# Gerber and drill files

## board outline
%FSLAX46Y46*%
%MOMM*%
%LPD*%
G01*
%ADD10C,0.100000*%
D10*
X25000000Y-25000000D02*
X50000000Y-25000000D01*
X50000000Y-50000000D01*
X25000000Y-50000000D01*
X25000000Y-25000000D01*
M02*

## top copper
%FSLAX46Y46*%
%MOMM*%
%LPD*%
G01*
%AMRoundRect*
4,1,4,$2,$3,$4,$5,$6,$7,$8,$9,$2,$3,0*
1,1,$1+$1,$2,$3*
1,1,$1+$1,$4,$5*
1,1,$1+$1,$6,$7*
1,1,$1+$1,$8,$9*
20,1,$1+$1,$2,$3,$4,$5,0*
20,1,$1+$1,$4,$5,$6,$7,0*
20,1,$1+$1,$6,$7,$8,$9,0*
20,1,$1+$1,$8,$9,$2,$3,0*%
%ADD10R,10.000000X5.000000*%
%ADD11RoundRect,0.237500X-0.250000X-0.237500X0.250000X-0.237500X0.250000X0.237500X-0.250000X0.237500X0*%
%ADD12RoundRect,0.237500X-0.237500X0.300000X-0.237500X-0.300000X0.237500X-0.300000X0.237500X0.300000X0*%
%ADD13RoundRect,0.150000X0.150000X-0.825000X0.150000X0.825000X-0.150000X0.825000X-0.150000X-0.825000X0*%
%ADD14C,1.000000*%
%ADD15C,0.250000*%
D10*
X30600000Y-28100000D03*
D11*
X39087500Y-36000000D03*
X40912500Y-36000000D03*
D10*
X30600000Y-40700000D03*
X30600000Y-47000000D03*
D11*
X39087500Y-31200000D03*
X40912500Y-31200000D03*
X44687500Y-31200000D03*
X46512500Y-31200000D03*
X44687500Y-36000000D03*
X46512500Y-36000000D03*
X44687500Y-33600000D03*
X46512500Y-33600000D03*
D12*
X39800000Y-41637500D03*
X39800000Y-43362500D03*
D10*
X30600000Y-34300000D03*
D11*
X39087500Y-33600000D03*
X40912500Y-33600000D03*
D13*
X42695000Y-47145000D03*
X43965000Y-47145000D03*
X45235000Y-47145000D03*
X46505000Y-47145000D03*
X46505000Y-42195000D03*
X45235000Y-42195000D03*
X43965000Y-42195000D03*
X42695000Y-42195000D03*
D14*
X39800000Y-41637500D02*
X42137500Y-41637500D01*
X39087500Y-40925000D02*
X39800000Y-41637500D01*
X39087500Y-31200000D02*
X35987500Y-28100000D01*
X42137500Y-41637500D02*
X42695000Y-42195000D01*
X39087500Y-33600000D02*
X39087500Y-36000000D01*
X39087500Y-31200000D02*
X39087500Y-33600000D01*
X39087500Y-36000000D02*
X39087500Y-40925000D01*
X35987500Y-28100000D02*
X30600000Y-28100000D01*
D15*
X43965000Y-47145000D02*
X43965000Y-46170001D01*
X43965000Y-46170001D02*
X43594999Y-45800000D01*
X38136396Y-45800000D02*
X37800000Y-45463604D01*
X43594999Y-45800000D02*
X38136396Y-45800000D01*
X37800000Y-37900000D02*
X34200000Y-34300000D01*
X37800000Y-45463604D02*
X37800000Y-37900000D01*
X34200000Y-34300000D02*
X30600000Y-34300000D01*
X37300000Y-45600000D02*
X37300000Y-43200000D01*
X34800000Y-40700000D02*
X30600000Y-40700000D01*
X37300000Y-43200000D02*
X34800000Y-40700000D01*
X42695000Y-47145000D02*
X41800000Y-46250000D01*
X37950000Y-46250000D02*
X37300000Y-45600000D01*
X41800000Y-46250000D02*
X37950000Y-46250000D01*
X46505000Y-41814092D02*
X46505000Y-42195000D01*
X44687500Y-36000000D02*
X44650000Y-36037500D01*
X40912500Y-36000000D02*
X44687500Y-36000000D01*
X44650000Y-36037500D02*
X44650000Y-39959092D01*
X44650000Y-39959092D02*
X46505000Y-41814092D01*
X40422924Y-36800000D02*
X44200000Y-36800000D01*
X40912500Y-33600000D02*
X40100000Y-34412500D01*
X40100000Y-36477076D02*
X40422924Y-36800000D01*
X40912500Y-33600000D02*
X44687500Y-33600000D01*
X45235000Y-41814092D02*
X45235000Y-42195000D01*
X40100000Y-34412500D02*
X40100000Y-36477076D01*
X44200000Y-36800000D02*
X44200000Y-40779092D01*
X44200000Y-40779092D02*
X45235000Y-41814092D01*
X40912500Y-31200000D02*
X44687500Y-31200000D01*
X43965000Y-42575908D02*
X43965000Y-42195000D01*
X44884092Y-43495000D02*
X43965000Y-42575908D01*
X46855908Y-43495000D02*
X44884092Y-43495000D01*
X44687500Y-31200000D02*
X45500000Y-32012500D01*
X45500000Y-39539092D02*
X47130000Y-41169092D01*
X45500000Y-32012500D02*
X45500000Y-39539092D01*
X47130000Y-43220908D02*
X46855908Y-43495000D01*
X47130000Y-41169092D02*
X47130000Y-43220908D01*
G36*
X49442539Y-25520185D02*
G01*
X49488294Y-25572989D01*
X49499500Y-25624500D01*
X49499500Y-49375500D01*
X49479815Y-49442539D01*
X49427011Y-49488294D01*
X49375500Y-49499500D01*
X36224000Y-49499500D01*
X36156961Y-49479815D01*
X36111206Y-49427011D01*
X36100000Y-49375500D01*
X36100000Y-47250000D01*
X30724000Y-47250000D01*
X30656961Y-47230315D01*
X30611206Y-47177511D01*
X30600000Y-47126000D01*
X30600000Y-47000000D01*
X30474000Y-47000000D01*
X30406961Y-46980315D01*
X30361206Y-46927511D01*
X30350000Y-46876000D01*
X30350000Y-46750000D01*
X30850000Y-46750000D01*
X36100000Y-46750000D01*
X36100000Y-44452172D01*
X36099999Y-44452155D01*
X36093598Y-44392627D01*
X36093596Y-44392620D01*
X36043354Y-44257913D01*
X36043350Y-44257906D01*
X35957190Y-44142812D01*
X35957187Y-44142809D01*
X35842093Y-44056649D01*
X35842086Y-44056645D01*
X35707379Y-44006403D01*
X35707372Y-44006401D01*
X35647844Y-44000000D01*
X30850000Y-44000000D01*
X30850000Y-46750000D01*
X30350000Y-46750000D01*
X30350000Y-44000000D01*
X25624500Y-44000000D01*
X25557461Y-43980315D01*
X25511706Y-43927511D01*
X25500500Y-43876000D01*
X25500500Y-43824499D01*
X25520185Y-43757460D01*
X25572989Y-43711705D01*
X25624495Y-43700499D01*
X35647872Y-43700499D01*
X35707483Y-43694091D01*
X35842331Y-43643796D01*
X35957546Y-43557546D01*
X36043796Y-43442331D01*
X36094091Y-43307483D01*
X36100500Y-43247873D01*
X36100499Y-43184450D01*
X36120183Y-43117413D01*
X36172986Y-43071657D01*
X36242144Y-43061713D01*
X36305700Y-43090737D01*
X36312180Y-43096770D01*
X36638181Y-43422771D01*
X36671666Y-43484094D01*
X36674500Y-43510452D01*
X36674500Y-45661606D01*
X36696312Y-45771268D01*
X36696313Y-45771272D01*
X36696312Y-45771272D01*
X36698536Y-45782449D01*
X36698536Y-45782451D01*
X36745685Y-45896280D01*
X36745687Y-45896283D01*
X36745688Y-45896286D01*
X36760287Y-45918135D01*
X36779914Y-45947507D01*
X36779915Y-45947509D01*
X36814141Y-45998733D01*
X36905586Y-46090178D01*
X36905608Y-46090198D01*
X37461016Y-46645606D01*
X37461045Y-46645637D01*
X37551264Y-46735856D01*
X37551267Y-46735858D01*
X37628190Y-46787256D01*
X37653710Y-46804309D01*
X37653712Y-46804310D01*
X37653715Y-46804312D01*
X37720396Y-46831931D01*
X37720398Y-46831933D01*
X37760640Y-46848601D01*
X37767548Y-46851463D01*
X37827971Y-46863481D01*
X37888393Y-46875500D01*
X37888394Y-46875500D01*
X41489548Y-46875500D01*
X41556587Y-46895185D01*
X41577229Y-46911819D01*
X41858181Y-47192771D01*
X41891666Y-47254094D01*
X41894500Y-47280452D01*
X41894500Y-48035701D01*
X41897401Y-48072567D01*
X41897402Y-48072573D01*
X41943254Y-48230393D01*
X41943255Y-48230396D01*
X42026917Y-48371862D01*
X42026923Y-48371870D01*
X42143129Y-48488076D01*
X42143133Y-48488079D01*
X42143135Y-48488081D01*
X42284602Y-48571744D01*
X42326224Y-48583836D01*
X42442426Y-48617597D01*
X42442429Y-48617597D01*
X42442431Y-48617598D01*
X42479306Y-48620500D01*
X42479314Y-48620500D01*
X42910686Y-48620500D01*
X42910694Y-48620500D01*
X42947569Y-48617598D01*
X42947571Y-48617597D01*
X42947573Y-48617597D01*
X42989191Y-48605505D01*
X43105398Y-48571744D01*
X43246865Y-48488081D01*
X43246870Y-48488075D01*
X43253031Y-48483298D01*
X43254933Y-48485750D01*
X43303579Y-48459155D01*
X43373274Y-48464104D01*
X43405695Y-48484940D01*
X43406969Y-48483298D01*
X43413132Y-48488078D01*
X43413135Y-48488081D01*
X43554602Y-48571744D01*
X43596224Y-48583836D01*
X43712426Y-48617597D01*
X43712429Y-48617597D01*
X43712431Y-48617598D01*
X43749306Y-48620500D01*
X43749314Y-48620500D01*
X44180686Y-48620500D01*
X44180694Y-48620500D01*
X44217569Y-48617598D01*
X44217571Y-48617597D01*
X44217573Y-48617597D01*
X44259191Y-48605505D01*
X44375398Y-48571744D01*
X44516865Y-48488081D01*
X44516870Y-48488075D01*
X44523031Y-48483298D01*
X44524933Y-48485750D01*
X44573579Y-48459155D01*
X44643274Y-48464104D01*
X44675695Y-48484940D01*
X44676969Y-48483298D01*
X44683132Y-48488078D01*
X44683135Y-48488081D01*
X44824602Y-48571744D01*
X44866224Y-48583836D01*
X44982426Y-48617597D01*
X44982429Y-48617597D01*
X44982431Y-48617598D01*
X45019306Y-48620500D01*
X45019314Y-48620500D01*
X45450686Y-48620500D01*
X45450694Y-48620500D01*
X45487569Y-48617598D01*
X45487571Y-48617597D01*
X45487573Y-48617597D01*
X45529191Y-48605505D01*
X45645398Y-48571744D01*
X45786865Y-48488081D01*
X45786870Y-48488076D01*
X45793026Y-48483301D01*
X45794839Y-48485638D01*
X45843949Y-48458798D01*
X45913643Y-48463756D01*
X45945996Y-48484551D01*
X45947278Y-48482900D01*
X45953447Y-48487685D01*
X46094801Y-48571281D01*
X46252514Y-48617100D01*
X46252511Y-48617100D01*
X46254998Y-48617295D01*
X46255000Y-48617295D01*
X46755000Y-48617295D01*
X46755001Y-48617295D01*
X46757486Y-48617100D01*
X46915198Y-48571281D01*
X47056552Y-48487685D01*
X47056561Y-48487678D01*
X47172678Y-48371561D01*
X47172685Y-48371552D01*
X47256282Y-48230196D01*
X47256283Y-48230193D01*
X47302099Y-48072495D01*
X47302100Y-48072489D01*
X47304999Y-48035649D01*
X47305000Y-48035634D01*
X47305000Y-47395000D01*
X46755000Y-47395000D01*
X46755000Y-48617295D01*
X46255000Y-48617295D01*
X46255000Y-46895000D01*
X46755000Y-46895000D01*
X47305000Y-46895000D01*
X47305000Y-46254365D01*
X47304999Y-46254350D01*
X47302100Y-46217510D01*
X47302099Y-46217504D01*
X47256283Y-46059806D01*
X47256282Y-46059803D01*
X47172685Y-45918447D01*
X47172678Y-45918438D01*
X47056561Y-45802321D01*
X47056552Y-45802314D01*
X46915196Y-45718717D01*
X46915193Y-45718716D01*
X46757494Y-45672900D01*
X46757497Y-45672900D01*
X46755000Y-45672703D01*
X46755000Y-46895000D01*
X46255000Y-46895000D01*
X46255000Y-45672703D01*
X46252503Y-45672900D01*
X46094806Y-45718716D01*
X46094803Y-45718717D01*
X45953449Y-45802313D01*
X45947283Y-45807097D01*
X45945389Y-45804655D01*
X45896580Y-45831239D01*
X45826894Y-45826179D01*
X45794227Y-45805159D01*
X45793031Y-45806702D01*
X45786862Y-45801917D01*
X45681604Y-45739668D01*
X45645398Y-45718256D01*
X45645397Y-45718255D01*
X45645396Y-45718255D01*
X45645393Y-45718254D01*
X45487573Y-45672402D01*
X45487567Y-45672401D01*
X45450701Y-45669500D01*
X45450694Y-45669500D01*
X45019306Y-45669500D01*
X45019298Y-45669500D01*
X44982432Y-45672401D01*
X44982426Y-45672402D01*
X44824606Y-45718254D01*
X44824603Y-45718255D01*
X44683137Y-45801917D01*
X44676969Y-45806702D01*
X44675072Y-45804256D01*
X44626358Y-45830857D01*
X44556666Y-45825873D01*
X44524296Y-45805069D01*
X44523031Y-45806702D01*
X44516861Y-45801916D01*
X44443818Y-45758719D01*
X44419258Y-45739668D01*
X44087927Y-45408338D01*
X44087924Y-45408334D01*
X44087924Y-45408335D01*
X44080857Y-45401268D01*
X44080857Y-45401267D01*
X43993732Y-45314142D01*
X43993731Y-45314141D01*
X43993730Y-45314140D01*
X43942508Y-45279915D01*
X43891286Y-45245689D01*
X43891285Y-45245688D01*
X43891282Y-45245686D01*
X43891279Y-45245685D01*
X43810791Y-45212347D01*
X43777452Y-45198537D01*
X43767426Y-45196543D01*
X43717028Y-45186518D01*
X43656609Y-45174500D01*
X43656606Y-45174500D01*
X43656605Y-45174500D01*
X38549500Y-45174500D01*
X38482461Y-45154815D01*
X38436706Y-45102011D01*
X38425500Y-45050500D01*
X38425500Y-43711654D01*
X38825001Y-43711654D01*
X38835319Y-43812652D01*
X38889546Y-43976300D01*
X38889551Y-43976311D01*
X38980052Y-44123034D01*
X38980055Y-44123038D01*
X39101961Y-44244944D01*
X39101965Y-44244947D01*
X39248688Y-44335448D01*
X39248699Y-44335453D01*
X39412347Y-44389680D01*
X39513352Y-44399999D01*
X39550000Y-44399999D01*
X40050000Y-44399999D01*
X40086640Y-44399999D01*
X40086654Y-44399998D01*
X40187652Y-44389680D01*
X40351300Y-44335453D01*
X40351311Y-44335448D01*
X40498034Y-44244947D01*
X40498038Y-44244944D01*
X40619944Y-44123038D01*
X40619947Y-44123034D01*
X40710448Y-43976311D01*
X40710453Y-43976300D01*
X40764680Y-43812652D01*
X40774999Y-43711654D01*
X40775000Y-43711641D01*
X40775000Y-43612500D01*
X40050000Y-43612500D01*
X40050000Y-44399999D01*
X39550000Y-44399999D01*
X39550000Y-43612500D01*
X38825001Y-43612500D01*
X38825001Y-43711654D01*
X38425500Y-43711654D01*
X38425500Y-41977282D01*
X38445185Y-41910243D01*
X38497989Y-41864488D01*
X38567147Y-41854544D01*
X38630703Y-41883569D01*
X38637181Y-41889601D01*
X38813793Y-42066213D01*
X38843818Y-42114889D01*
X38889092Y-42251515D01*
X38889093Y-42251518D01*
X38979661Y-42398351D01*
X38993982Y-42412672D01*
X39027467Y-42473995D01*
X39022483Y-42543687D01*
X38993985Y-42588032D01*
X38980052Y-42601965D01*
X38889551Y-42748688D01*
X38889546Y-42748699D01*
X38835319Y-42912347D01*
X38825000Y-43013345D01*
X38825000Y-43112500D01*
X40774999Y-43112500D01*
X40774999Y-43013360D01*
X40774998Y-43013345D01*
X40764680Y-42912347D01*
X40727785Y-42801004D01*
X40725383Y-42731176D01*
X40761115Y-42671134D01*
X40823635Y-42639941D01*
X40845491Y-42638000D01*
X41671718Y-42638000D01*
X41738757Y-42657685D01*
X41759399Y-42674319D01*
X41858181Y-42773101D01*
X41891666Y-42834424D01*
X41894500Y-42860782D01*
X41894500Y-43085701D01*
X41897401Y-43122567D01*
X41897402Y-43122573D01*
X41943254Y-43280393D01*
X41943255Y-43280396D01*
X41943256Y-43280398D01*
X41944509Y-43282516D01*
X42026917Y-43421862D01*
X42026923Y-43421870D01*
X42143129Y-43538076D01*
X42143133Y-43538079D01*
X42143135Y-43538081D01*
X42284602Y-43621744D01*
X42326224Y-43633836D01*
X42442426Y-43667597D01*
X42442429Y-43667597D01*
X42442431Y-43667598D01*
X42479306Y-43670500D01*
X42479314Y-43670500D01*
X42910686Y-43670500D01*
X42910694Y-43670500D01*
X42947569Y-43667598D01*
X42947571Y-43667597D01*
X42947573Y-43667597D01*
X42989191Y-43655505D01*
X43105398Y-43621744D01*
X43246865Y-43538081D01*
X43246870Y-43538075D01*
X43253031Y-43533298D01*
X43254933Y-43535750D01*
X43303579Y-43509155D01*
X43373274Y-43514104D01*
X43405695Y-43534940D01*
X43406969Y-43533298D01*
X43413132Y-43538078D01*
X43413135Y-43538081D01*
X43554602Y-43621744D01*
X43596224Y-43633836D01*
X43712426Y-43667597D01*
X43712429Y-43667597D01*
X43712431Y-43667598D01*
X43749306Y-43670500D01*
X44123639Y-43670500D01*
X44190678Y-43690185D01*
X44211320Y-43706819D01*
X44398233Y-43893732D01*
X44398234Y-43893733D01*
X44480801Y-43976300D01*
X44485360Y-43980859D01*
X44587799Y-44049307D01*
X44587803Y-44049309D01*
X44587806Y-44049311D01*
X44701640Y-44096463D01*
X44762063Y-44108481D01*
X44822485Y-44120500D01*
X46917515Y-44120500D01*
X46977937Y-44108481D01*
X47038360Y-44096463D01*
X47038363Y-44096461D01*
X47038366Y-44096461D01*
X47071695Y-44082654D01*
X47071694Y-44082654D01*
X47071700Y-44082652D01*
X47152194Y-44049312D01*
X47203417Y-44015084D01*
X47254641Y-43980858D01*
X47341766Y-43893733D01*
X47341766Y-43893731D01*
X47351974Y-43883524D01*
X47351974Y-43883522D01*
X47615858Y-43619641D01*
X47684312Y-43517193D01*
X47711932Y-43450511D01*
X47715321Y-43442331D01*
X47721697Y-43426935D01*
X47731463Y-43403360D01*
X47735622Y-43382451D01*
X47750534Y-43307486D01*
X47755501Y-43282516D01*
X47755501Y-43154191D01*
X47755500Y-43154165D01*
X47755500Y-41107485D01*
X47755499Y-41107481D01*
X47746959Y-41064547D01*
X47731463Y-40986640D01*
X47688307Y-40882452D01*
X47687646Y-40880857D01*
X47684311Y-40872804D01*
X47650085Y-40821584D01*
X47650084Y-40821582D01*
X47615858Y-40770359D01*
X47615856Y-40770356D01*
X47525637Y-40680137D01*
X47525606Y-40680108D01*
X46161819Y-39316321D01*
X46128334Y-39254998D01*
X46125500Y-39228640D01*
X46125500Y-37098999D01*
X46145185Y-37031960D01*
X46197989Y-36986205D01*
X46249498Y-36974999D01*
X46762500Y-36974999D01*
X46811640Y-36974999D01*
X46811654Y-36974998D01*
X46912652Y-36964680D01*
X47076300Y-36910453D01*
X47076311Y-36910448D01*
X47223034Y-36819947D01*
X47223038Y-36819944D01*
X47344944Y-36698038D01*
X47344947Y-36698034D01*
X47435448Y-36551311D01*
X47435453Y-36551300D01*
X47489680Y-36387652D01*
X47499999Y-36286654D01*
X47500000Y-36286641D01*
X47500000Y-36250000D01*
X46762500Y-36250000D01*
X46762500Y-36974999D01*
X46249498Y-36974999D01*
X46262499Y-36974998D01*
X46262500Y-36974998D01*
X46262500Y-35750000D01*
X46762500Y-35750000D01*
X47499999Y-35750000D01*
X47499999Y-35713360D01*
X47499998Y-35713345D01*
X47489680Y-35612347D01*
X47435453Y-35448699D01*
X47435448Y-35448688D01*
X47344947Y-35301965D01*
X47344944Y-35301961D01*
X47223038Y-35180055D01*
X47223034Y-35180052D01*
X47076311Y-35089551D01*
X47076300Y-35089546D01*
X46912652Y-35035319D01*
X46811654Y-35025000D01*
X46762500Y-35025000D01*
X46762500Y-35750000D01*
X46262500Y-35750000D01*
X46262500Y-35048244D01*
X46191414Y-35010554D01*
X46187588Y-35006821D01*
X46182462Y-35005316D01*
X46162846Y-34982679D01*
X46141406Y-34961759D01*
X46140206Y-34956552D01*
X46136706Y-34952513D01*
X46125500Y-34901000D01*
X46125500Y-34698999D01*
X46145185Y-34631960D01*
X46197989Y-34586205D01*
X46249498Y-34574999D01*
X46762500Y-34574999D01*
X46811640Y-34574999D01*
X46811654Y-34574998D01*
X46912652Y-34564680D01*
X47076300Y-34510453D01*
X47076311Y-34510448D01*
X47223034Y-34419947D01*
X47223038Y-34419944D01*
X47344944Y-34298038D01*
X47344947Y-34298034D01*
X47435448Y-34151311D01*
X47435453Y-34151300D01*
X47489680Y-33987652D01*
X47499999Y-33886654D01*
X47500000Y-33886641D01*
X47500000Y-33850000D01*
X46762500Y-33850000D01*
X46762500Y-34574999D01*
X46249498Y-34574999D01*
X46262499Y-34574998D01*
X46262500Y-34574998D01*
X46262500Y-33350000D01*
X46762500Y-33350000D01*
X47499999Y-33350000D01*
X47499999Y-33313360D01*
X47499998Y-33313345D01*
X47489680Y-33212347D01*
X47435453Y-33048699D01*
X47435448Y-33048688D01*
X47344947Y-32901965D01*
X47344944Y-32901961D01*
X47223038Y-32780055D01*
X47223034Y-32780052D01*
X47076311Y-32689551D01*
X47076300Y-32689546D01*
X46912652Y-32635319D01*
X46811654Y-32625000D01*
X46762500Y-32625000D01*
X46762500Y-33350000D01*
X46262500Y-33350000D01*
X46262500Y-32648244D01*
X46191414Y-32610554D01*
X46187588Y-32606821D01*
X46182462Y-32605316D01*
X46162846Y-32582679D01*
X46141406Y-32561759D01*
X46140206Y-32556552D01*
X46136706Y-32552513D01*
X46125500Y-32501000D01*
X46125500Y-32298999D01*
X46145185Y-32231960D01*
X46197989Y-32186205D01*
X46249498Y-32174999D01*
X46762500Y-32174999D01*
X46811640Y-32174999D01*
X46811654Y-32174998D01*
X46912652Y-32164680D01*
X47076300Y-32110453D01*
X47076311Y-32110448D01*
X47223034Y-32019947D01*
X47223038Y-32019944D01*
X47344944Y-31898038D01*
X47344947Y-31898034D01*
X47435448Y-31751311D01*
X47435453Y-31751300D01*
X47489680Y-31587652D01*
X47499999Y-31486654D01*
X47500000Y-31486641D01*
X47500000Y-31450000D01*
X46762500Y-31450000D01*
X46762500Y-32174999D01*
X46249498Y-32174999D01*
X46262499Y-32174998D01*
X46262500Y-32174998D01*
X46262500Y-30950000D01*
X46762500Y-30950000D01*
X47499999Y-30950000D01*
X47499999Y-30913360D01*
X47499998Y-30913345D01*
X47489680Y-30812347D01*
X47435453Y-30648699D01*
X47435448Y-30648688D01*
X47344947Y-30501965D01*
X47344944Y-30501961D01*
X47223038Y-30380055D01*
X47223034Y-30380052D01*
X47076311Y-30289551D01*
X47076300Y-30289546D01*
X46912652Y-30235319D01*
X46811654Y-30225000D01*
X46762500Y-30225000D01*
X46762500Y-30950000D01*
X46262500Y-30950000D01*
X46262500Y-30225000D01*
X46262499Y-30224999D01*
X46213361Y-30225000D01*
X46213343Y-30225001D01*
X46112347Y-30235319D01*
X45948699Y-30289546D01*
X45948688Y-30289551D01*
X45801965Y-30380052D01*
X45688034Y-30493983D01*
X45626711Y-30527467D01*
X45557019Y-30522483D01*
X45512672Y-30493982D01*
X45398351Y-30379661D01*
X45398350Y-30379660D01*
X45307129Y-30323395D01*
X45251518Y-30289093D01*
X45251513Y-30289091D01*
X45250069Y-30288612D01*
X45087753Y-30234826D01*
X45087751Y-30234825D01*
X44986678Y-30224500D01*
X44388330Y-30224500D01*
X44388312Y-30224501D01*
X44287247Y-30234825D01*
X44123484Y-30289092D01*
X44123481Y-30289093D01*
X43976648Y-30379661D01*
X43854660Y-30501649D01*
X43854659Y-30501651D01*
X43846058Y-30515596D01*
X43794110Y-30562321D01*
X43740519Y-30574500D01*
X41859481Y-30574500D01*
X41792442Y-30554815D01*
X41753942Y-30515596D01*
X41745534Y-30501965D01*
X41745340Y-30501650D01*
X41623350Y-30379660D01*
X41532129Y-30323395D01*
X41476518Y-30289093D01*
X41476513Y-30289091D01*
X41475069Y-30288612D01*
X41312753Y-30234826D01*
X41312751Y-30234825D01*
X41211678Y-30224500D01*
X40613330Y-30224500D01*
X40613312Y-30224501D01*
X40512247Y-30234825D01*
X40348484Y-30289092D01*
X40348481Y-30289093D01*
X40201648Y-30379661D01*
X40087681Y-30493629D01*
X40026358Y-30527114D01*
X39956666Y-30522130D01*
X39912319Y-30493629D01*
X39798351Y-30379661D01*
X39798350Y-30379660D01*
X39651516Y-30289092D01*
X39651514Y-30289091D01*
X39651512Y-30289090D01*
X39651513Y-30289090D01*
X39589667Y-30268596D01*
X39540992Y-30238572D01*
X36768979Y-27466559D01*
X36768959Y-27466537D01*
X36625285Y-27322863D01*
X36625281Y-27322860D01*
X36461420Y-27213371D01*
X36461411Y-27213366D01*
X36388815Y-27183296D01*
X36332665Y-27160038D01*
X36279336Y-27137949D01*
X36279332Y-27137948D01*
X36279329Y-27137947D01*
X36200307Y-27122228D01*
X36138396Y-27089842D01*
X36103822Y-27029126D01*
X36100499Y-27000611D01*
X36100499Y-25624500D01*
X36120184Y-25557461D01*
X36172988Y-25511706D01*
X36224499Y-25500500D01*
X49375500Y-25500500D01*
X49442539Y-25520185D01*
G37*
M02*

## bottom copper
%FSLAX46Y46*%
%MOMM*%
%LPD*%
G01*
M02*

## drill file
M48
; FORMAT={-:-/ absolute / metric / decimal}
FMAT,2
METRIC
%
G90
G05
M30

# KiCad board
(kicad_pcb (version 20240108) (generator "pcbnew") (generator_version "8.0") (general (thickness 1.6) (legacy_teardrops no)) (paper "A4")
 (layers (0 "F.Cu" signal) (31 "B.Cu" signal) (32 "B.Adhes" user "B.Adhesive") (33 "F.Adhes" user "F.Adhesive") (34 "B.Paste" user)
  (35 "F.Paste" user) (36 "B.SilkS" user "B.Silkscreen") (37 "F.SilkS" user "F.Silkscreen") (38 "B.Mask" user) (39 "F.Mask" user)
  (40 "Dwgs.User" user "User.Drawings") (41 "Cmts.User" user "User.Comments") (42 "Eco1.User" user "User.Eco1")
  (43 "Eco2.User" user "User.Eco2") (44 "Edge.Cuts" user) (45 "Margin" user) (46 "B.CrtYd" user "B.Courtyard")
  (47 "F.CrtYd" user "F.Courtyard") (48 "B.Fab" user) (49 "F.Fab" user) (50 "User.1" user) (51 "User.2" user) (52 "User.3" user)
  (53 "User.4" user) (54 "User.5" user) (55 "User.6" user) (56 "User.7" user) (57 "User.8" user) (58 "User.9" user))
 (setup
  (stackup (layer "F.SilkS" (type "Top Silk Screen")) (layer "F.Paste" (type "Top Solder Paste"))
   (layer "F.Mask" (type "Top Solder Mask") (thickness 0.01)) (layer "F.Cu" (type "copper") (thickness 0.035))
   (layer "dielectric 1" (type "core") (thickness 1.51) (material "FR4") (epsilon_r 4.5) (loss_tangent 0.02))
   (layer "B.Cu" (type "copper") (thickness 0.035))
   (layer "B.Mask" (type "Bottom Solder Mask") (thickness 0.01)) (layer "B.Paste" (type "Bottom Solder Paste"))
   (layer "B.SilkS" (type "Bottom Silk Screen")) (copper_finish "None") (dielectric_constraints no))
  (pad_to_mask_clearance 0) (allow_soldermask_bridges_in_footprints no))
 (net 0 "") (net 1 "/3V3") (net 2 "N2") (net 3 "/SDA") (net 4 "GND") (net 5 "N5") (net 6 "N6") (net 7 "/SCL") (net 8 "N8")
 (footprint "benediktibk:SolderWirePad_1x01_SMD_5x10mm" (layer "F.Cu") (at 30.6 28.1 -90)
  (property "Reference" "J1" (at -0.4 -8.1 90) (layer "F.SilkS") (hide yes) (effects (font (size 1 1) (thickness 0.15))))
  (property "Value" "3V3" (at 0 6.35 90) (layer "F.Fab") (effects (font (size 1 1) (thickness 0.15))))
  (pad "1" smd rect (at 0 0 270) (size 5 10) (layers "F.Cu" "F.Paste" "F.Mask") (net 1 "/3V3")))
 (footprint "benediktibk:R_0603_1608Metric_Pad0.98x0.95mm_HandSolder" (layer "F.Cu") (at 40 36)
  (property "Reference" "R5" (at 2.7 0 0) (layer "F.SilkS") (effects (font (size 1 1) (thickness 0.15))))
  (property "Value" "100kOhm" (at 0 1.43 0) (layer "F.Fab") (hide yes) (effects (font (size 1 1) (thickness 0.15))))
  (pad "1" smd roundrect (at -0.9125 0) (size 0.975 0.95) (layers "F.Cu" "F.Paste" "F.Mask") (roundrect_rratio 0.25) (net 1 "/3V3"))
  (pad "2" smd roundrect (at 0.9125 0) (size 0.975 0.95) (layers "F.Cu" "F.Paste" "F.Mask") (roundrect_rratio 0.25) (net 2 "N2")))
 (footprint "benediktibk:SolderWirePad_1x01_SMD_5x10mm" (layer "F.Cu") (at 30.6 40.7 -90)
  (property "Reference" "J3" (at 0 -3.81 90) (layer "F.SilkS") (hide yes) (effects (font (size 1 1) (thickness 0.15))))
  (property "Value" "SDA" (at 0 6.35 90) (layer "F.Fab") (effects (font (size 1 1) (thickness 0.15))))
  (pad "1" smd rect (at 0 0 270) (size 5 10) (layers "F.Cu" "F.Paste" "F.Mask") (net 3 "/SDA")))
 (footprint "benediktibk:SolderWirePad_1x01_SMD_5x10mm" (layer "F.Cu") (at 30.6 47 -90)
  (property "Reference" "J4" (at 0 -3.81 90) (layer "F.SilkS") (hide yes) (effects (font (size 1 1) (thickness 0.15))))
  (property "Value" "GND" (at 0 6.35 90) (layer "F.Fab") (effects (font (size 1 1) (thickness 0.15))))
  (pad "1" smd rect (at 0 0 270) (size 5 10) (layers "F.Cu" "F.Paste" "F.Mask") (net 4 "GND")))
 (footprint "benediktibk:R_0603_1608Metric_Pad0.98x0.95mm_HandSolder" (layer "F.Cu") (at 40 31.2)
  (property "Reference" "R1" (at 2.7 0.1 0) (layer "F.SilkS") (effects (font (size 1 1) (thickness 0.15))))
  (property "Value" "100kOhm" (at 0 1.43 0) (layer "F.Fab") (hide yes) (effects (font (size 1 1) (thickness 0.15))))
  (pad "1" smd roundrect (at -0.9125 0) (size 0.975 0.95) (layers "F.Cu" "F.Paste" "F.Mask") (roundrect_rratio 0.25) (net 1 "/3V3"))
  (pad "2" smd roundrect (at 0.9125 0) (size 0.975 0.95) (layers "F.Cu" "F.Paste" "F.Mask") (roundrect_rratio 0.25) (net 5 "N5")))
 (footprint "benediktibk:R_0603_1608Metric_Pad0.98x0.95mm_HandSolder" (layer "F.Cu") (at 45.6 31.2)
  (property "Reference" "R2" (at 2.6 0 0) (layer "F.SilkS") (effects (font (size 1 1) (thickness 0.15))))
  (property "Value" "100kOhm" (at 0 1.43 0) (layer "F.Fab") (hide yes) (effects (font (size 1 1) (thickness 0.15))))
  (pad "1" smd roundrect (at -0.9125 0) (size 0.975 0.95) (layers "F.Cu" "F.Paste" "F.Mask") (roundrect_rratio 0.25) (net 5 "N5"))
  (pad "2" smd roundrect (at 0.9125 0) (size 0.975 0.95) (layers "F.Cu" "F.Paste" "F.Mask") (roundrect_rratio 0.25) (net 4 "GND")))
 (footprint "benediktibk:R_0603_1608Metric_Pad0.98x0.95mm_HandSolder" (layer "F.Cu") (at 45.6 36)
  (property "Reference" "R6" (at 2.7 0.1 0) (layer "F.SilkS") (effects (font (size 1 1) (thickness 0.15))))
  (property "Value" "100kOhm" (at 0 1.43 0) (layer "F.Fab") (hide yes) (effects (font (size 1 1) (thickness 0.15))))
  (pad "1" smd roundrect (at -0.9125 0) (size 0.975 0.95) (layers "F.Cu" "F.Paste" "F.Mask") (roundrect_rratio 0.25) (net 2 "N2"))
  (pad "2" smd roundrect (at 0.9125 0) (size 0.975 0.95) (layers "F.Cu" "F.Paste" "F.Mask") (roundrect_rratio 0.25) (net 4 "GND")))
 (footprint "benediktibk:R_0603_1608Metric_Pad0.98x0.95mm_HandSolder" (layer "F.Cu") (at 45.6 33.6)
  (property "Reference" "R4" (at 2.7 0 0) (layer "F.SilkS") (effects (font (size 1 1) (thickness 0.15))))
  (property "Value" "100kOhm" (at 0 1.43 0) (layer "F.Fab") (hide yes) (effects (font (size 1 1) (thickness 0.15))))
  (pad "1" smd roundrect (at -0.9125 0) (size 0.975 0.95) (layers "F.Cu" "F.Paste" "F.Mask") (roundrect_rratio 0.25) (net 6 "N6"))
  (pad "2" smd roundrect (at 0.9125 0) (size 0.975 0.95) (layers "F.Cu" "F.Paste" "F.Mask") (roundrect_rratio 0.25) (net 4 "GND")))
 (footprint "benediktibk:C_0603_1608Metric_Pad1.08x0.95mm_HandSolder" (layer "F.Cu") (at 39.8 42.5 -90)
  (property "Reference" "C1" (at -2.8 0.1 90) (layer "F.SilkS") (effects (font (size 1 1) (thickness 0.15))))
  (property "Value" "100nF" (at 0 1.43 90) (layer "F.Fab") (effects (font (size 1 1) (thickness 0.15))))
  (pad "1" smd roundrect (at -0.8625 0 270) (size 1.075 0.95) (layers "F.Cu" "F.Paste" "F.Mask") (roundrect_rratio 0.25) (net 1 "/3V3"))
  (pad "2" smd roundrect (at 0.8625 0 270) (size 1.075 0.95) (layers "F.Cu" "F.Paste" "F.Mask") (roundrect_rratio 0.25) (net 4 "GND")))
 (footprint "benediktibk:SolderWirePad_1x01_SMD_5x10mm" (layer "F.Cu") (at 30.6 34.3 -90)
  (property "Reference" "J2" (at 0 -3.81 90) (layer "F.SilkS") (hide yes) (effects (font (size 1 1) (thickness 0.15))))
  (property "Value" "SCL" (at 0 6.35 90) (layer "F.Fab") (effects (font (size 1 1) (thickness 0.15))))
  (pad "1" smd rect (at 0 0 270) (size 5 10) (layers "F.Cu" "F.Paste" "F.Mask") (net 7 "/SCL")))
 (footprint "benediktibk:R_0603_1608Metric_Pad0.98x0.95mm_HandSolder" (layer "F.Cu") (at 40 33.6)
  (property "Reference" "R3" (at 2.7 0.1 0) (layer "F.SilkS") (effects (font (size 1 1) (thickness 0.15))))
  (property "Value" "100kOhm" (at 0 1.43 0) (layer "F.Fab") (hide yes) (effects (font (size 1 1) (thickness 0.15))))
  (pad "1" smd roundrect (at -0.9125 0) (size 0.975 0.95) (layers "F.Cu" "F.Paste" "F.Mask") (roundrect_rratio 0.25) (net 1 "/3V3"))
  (pad "2" smd roundrect (at 0.9125 0) (size 0.975 0.95) (layers "F.Cu" "F.Paste" "F.Mask") (roundrect_rratio 0.25) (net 6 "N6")))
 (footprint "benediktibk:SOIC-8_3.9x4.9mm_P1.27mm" (layer "F.Cu") (at 44.6 44.67 90)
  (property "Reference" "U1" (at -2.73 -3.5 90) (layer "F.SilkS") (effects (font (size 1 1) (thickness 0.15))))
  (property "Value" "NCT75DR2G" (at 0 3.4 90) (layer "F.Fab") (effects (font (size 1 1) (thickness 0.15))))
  (pad "1" smd roundrect (at -2.475 -1.905 90) (size 1.95 0.6) (layers "F.Cu" "F.Paste" "F.Mask") (roundrect_rratio 0.25) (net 3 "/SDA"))
  (pad "2" smd roundrect (at -2.475 -0.635 90) (size 1.95 0.6) (layers "F.Cu" "F.Paste" "F.Mask") (roundrect_rratio 0.25) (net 7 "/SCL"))
  (pad "3" smd roundrect (at -2.475 0.635 90) (size 1.95 0.6) (layers "F.Cu" "F.Paste" "F.Mask") (roundrect_rratio 0.25) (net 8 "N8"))
  (pad "4" smd roundrect (at -2.475 1.905 90) (size 1.95 0.6) (layers "F.Cu" "F.Paste" "F.Mask") (roundrect_rratio 0.25) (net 4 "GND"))
  (pad "5" smd roundrect (at 2.475 1.905 90) (size 1.95 0.6) (layers "F.Cu" "F.Paste" "F.Mask") (roundrect_rratio 0.25) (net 2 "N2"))
  (pad "6" smd roundrect (at 2.475 0.635 90) (size 1.95 0.6) (layers "F.Cu" "F.Paste" "F.Mask") (roundrect_rratio 0.25) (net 6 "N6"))
  (pad "7" smd roundrect (at 2.475 -0.635 90) (size 1.95 0.6) (layers "F.Cu" "F.Paste" "F.Mask") (roundrect_rratio 0.25) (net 5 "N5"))
  (pad "8" smd roundrect (at 2.475 -1.905 90) (size 1.95 0.6) (layers "F.Cu" "F.Paste" "F.Mask") (roundrect_rratio 0.25) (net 1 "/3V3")))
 (gr_rect (start 25 25) (end 50 50) (stroke (width 0.1) (type default)) (fill none) (layer "Edge.Cuts"))
 (segment (start 39.8 41.6375) (end 42.1375 41.6375) (width 1) (layer "F.Cu") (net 1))
 (segment (start 39.0875 40.925) (end 39.8 41.6375) (width 1) (layer "F.Cu") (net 1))
 (segment (start 39.0875 31.2) (end 35.9875 28.1) (width 1) (layer "F.Cu") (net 1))
 (segment (start 42.1375 41.6375) (end 42.695 42.195) (width 1) (layer "F.Cu") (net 1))
 (segment (start 39.0875 33.6) (end 39.0875 36) (width 1) (layer "F.Cu") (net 1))
 (segment (start 39.0875 31.2) (end 39.0875 33.6) (width 1) (layer "F.Cu") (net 1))
 (segment (start 39.0875 36) (end 39.0875 40.925) (width 1) (layer "F.Cu") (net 1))
 (segment (start 35.9875 28.1) (end 30.6 28.1) (width 1) (layer "F.Cu") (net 1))
 (segment (start 43.965 47.145) (end 43.965 46.170001) (width 0.25) (layer "F.Cu") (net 7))
 (segment (start 43.965 46.170001) (end 43.594999 45.8) (width 0.25) (layer "F.Cu") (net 7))
 (segment (start 38.136396 45.8) (end 37.8 45.463604) (width 0.25) (layer "F.Cu") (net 7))
 (segment (start 43.594999 45.8) (end 38.136396 45.8) (width 0.25) (layer "F.Cu") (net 7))
 (segment (start 37.8 37.9) (end 34.2 34.3) (width 0.25) (layer "F.Cu") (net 7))
 (segment (start 37.8 45.463604) (end 37.8 37.9) (width 0.25) (layer "F.Cu") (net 7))
 (segment (start 34.2 34.3) (end 30.6 34.3) (width 0.25) (layer "F.Cu") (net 7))
 (segment (start 37.3 45.6) (end 37.3 43.2) (width 0.25) (layer "F.Cu") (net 3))
 (segment (start 34.8 40.7) (end 30.6 40.7) (width 0.25) (layer "F.Cu") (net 3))
 (segment (start 37.3 43.2) (end 34.8 40.7) (width 0.25) (layer "F.Cu") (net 3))
 (segment (start 42.695 47.145) (end 41.8 46.25) (width 0.25) (layer "F.Cu") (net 3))
 (segment (start 37.95 46.25) (end 37.3 45.6) (width 0.25) (layer "F.Cu") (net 3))
 (segment (start 41.8 46.25) (end 37.95 46.25) (width 0.25) (layer "F.Cu") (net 3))
 (segment (start 46.505 41.814092) (end 46.505 42.195) (width 0.25) (layer "F.Cu") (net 2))
 (segment (start 44.6875 36) (end 44.65 36.0375) (width 0.25) (layer "F.Cu") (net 2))
 (segment (start 40.9125 36) (end 44.6875 36) (width 0.25) (layer "F.Cu") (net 2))
 (segment (start 44.65 36.0375) (end 44.65 39.959092) (width 0.25) (layer "F.Cu") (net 2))
 (segment (start 44.65 39.959092) (end 46.505 41.814092) (width 0.25) (layer "F.Cu") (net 2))
 (segment (start 40.422924 36.8) (end 44.2 36.8) (width 0.25) (layer "F.Cu") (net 6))
 (segment (start 40.9125 33.6) (end 40.1 34.4125) (width 0.25) (layer "F.Cu") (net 6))
 (segment (start 40.1 36.477076) (end 40.422924 36.8) (width 0.25) (layer "F.Cu") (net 6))
 (segment (start 40.9125 33.6) (end 44.6875 33.6) (width 0.25) (layer "F.Cu") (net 6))
 (segment (start 45.235 41.814092) (end 45.235 42.195) (width 0.25) (layer "F.Cu") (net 6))
 (segment (start 40.1 34.4125) (end 40.1 36.477076) (width 0.25) (layer "F.Cu") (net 6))
 (segment (start 44.2 36.8) (end 44.2 40.779092) (width 0.25) (layer "F.Cu") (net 6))
 (segment (start 44.2 40.779092) (end 45.235 41.814092) (width 0.25) (layer "F.Cu") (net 6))
 (segment (start 40.9125 31.2) (end 44.6875 31.2) (width 0.25) (layer "F.Cu") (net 5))
 (segment (start 43.965 42.575908) (end 43.965 42.195) (width 0.25) (layer "F.Cu") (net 5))
 (segment (start 44.884092 43.495) (end 43.965 42.575908) (width 0.25) (layer "F.Cu") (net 5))
 (segment (start 46.855908 43.495) (end 44.884092 43.495) (width 0.25) (layer "F.Cu") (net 5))
 (segment (start 44.6875 31.2) (end 45.5 32.0125) (width 0.25) (layer "F.Cu") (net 5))
 (segment (start 45.5 39.539092) (end 47.13 41.169092) (width 0.25) (layer "F.Cu") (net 5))
 (segment (start 45.5 32.0125) (end 45.5 39.539092) (width 0.25) (layer "F.Cu") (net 5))
 (segment (start 47.13 43.220908) (end 46.855908 43.495) (width 0.25) (layer "F.Cu") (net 5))
 (segment (start 47.13 41.169092) (end 47.13 43.220908) (width 0.25) (layer "F.Cu") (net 5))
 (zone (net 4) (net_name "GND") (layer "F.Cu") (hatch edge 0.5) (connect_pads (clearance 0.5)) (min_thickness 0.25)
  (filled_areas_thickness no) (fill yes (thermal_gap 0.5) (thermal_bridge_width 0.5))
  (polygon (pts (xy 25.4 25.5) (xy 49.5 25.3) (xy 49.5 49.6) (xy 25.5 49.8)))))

